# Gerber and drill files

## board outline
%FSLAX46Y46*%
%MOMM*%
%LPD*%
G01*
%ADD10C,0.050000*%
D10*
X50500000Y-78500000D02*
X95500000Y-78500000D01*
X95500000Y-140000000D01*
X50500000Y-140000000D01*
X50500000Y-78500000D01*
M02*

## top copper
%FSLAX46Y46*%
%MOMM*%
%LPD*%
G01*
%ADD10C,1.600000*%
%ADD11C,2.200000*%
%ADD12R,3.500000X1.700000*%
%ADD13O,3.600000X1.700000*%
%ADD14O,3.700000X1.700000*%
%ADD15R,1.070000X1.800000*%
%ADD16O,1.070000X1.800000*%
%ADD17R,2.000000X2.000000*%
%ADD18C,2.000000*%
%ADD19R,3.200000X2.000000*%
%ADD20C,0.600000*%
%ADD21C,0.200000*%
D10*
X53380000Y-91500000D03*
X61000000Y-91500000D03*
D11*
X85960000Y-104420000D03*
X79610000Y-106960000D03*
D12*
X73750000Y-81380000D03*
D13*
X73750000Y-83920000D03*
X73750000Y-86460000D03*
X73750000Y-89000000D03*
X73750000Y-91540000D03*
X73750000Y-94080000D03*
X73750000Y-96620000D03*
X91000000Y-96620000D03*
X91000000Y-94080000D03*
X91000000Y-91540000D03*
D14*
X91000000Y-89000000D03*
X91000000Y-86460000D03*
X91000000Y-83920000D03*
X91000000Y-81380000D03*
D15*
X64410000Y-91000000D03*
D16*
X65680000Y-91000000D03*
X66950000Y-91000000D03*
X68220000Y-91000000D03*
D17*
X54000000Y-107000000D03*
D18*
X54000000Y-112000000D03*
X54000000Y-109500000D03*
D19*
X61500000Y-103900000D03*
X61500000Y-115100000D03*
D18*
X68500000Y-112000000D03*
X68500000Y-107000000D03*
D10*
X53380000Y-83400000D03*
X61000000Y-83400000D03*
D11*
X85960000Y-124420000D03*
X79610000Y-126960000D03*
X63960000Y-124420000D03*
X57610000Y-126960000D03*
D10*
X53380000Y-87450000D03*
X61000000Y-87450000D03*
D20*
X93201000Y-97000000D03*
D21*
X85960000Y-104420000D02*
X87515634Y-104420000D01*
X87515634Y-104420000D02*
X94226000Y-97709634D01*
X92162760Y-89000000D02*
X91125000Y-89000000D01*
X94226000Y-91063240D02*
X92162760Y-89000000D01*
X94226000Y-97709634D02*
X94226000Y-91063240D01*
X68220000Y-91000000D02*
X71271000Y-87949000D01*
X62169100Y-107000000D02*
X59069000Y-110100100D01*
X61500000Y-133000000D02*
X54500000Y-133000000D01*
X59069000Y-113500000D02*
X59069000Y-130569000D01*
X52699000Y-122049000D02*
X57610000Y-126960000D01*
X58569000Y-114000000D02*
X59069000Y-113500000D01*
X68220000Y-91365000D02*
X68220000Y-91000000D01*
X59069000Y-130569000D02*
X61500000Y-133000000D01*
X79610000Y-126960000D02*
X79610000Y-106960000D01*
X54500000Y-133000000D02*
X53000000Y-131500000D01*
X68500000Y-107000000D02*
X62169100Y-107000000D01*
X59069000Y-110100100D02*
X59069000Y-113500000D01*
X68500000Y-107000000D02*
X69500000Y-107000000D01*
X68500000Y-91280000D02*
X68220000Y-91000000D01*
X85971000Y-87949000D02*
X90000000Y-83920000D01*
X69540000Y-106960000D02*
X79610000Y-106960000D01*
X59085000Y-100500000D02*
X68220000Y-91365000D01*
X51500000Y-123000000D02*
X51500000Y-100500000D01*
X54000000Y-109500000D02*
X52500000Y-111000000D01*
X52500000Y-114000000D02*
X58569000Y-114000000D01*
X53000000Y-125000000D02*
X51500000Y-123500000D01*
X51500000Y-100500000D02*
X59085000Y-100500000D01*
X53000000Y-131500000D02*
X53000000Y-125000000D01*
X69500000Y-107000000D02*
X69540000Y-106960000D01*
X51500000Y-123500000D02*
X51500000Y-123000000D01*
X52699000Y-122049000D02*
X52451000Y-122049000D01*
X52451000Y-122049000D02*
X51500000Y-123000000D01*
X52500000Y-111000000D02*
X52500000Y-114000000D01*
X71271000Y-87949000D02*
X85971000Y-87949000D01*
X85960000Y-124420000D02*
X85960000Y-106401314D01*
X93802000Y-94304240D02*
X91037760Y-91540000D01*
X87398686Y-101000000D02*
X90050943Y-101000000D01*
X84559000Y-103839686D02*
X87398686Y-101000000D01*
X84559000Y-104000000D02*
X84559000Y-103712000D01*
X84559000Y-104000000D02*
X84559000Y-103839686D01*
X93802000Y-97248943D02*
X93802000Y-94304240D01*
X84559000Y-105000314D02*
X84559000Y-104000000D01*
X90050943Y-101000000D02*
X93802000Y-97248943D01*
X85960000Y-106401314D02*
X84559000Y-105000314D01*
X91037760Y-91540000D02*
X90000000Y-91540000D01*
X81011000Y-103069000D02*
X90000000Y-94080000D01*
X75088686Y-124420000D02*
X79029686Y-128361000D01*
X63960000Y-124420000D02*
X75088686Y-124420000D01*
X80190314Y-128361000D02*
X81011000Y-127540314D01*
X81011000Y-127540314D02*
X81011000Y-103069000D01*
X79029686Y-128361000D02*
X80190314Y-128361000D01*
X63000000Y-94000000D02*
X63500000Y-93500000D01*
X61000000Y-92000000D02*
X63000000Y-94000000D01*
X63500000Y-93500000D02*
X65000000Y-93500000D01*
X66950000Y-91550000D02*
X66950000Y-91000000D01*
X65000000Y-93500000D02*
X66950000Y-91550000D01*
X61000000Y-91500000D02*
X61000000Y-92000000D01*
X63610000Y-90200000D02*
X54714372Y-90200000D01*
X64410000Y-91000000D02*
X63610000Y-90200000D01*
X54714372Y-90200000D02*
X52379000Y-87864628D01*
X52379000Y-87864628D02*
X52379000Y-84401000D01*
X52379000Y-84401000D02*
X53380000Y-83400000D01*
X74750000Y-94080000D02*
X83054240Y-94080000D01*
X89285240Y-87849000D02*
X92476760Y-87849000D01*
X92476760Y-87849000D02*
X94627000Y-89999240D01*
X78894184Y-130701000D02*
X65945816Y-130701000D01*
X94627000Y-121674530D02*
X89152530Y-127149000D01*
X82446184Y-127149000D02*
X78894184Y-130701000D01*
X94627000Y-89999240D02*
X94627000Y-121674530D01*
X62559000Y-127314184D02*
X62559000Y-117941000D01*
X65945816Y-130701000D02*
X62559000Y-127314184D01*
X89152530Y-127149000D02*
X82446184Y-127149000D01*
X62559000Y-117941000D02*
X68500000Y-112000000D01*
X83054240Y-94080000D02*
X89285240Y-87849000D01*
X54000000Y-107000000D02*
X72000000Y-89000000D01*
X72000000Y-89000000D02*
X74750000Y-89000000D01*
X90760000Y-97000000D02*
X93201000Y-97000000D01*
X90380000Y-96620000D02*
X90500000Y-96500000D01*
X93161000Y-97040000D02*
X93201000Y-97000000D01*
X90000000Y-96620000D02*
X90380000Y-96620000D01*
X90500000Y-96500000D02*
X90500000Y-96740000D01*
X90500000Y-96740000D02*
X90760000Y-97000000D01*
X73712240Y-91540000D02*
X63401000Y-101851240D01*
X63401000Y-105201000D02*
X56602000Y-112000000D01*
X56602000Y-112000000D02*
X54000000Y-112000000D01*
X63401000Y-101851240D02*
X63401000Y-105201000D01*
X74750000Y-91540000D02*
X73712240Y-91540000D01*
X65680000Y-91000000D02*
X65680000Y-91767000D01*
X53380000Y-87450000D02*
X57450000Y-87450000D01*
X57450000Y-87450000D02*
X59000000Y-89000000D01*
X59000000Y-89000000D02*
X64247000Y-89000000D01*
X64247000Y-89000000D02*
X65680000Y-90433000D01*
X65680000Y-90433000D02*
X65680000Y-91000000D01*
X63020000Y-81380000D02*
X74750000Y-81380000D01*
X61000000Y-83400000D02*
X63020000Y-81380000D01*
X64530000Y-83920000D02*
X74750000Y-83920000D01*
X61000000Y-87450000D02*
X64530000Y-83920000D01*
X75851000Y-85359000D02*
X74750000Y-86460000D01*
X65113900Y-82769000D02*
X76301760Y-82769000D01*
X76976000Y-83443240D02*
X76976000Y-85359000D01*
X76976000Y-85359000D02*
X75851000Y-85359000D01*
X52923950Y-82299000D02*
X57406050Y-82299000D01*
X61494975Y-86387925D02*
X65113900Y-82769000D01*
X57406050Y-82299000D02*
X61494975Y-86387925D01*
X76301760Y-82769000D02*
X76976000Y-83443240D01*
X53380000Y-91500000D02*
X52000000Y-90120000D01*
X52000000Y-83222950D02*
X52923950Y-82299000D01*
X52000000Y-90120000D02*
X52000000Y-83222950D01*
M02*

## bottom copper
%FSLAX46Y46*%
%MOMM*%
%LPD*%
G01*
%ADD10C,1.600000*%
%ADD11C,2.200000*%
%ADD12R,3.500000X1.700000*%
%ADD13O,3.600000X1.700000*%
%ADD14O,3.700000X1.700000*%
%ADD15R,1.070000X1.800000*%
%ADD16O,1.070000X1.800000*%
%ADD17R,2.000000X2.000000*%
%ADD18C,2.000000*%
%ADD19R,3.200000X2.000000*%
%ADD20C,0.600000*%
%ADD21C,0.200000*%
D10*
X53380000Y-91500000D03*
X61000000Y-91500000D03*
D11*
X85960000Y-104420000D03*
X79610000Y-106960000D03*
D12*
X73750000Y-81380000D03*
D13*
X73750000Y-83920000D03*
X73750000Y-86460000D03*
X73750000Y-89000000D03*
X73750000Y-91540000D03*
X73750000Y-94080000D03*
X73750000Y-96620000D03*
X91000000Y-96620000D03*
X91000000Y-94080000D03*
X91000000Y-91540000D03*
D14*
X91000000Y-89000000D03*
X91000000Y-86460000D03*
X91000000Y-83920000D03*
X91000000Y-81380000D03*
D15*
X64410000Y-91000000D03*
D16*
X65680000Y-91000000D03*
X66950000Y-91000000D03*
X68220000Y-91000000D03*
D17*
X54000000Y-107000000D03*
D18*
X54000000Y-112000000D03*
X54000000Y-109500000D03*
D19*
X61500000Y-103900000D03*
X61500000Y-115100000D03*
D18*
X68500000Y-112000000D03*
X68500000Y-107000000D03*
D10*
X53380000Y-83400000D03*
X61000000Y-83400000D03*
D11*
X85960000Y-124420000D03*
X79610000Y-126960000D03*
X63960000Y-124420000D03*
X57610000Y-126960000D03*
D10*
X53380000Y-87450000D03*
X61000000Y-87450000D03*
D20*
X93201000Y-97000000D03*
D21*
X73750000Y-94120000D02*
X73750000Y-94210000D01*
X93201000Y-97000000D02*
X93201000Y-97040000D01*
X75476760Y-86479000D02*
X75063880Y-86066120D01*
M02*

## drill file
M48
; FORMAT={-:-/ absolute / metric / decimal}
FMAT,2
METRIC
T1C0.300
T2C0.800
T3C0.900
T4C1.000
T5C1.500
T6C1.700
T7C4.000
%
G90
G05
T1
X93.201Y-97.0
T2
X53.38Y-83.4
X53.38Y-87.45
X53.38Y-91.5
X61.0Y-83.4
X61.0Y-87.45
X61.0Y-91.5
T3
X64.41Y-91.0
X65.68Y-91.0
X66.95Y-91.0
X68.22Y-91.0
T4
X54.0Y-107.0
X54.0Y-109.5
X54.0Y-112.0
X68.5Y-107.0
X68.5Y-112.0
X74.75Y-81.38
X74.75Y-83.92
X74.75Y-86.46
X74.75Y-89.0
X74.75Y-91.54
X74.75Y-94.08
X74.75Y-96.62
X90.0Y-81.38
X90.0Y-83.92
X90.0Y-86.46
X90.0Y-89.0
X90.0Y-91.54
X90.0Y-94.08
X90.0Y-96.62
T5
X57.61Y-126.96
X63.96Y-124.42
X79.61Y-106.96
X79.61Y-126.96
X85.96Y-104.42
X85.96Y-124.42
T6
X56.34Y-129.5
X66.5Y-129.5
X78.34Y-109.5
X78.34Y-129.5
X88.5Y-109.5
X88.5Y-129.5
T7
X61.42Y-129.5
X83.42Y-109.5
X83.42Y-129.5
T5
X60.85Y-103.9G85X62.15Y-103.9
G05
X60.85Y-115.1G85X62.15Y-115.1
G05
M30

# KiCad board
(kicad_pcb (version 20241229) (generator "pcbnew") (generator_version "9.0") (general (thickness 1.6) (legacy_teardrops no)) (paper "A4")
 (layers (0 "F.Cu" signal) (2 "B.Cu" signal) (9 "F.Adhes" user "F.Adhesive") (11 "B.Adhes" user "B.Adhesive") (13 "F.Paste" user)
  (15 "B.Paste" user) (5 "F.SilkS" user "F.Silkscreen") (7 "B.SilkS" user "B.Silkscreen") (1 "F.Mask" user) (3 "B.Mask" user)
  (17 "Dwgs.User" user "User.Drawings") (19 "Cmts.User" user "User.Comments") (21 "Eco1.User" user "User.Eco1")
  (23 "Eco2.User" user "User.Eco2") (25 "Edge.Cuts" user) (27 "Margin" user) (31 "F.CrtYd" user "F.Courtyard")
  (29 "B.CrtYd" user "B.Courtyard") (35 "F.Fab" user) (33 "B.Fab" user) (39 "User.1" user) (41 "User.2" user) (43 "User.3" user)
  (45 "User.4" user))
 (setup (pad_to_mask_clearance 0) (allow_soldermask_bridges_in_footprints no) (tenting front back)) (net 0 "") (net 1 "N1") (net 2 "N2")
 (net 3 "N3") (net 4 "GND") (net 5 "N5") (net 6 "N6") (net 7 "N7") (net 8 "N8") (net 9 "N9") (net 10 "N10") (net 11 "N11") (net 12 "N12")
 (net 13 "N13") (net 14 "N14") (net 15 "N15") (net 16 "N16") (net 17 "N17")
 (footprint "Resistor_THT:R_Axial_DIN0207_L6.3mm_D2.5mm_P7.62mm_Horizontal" (layer "F.Cu") (at 53.38 91.5)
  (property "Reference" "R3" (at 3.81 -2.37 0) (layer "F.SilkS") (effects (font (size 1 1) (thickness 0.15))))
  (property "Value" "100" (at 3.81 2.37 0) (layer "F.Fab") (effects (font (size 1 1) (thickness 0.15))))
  (pad "1" thru_hole circle (at 0 0) (size 1.6 1.6) (drill 0.8) (layers "*.Cu" "*.Mask") (remove_unused_layers no) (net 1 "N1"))
  (pad "2" thru_hole circle (at 7.62 0) (size 1.6 1.6) (drill 0.8) (layers "*.Cu" "*.Mask") (remove_unused_layers no) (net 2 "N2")))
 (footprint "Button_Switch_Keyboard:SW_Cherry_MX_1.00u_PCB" (layer "F.Cu") (at 85.96 104.42)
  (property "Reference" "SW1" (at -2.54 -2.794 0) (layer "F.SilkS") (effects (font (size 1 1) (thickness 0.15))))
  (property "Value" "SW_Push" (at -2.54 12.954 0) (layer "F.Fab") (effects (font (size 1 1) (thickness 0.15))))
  (pad "" np_thru_hole circle (at -7.62 5.08) (size 1.7 1.7) (drill 1.7) (layers "*.Cu" "*.Mask"))
  (pad "" np_thru_hole circle (at -2.54 5.08) (size 4 4) (drill 4) (layers "*.Cu" "*.Mask"))
  (pad "" np_thru_hole circle (at 2.54 5.08) (size 1.7 1.7) (drill 1.7) (layers "*.Cu" "*.Mask"))
  (pad "1" thru_hole circle (at 0 0) (size 2.2 2.2) (drill 1.5) (layers "*.Cu" "*.Mask") (remove_unused_layers no) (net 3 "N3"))
  (pad "2" thru_hole circle (at -6.35 2.54) (size 2.2 2.2) (drill 1.5) (layers "*.Cu" "*.Mask") (remove_unused_layers no) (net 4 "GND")))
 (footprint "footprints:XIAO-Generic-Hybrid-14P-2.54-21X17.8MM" (layer "F.Cu") (at 82.375 89)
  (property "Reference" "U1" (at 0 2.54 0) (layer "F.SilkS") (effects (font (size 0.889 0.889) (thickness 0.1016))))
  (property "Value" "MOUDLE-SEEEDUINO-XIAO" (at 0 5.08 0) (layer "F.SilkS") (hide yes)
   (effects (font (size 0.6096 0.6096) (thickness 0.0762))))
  (pad "1" thru_hole rect (at -7.625 -7.62) (size 3.5 1.7) (drill 1 (offset -1 0)) (layers "*.Cu" "*.Mask") (remove_unused_layers no)
   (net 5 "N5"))
  (pad "2" thru_hole oval (at -7.625 -5.08) (size 3.6 1.7) (drill 1 (offset -1 0)) (layers "*.Cu" "*.Mask") (remove_unused_layers no)
   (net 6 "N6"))
  (pad "3" thru_hole oval (at -7.625 -2.54) (size 3.6 1.7) (drill 1 (offset -1 0)) (layers "*.Cu" "*.Mask") (remove_unused_layers no)
   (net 1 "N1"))
  (pad "4" thru_hole oval (at -7.625 0) (size 3.6 1.7) (drill 1 (offset -1 0)) (layers "*.Cu" "*.Mask") (remove_unused_layers no)
   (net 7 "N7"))
  (pad "5" thru_hole oval (at -7.625 2.54) (size 3.6 1.7) (drill 1 (offset -1 0)) (layers "*.Cu" "*.Mask") (remove_unused_layers no)
   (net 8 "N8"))
  (pad "6" thru_hole oval (at -7.625 5.08 180) (size 3.6 1.7) (drill 1 (offset 1 0)) (layers "*.Cu" "*.Mask") (remove_unused_layers no)
   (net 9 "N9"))
  (pad "7" thru_hole oval (at -7.625 7.62) (size 3.6 1.7) (drill 1 (offset -1 0)) (layers "*.Cu" "*.Mask") (remove_unused_layers no)
   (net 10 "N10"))
  (pad "8" thru_hole oval (at 7.625 7.62) (size 3.6 1.7) (drill 1 (offset 1 0)) (layers "*.Cu" "*.Mask") (remove_unused_layers no)
   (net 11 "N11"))
  (pad "9" thru_hole oval (at 7.625 5.08) (size 3.6 1.7) (drill 1 (offset 1 0)) (layers "*.Cu" "*.Mask") (remove_unused_layers no)
   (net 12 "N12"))
  (pad "10" thru_hole oval (at 7.625 2.54) (size 3.6 1.7) (drill 1 (offset 1 0)) (layers "*.Cu" "*.Mask") (remove_unused_layers no)
   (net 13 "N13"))
  (pad "11" thru_hole oval (at 7.625 0) (size 3.7 1.7) (drill 1 (offset 1 0)) (layers "*.Cu" "*.Mask") (remove_unused_layers no)
   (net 3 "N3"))
  (pad "12" thru_hole oval (at 7.625 -2.54) (size 3.7 1.7) (drill 1 (offset 1 0)) (layers "*.Cu" "*.Mask") (remove_unused_layers no)
   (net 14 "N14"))
  (pad "13" thru_hole oval (at 7.625 -5.08) (size 3.7 1.7) (drill 1 (offset 1 0)) (layers "*.Cu" "*.Mask") (remove_unused_layers no)
   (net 4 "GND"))
  (pad "14" thru_hole oval (at 7.625 -7.62) (size 3.7 1.7) (drill 1 (offset 1 0)) (layers "*.Cu" "*.Mask") (remove_unused_layers no)
   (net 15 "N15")))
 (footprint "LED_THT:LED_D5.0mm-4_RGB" (layer "F.Cu") (at 64.41 91)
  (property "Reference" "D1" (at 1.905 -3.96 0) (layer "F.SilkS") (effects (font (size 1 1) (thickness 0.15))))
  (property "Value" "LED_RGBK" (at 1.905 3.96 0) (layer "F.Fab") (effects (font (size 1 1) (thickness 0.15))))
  (pad "1" thru_hole rect (at 0 0) (size 1.07 1.8) (drill 0.9) (layers "*.Cu" "*.Mask") (remove_unused_layers no) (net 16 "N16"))
  (pad "2" thru_hole oval (at 1.27 0) (size 1.07 1.8) (drill 0.9) (layers "*.Cu" "*.Mask") (remove_unused_layers no) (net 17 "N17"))
  (pad "3" thru_hole oval (at 2.54 0) (size 1.07 1.8) (drill 0.9) (layers "*.Cu" "*.Mask") (remove_unused_layers no) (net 2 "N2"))
  (pad "4" thru_hole oval (at 3.81 0) (size 1.07 1.8) (drill 0.9) (layers "*.Cu" "*.Mask") (remove_unused_layers no) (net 4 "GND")))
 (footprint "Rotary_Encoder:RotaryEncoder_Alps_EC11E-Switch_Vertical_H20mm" (layer "F.Cu") (at 54 107)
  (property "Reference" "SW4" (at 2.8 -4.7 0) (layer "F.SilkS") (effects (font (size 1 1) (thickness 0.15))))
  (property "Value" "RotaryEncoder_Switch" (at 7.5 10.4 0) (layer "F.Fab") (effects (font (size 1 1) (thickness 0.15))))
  (pad "A" thru_hole rect (at 0 0) (size 2 2) (drill 1) (layers "*.Cu" "*.Mask") (remove_unused_layers no) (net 7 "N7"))
  (pad "B" thru_hole circle (at 0 5) (size 2 2) (drill 1) (layers "*.Cu" "*.Mask") (remove_unused_layers no) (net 8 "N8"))
  (pad "C" thru_hole circle (at 0 2.5) (size 2 2) (drill 1) (layers "*.Cu" "*.Mask") (remove_unused_layers no) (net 4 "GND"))
  (pad "MP" thru_hole rect (at 7.5 -3.1) (size 3.2 2) (drill oval 2.8 1.5) (layers "*.Cu" "*.Mask") (remove_unused_layers no))
  (pad "MP" thru_hole rect (at 7.5 8.1) (size 3.2 2) (drill oval 2.8 1.5) (layers "*.Cu" "*.Mask") (remove_unused_layers no))
  (pad "S1" thru_hole circle (at 14.5 5) (size 2 2) (drill 1) (layers "*.Cu" "*.Mask") (remove_unused_layers no) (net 9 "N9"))
  (pad "S2" thru_hole circle (at 14.5 0) (size 2 2) (drill 1) (layers "*.Cu" "*.Mask") (remove_unused_layers no) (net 4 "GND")))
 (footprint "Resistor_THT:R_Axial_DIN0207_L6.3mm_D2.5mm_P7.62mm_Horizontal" (layer "F.Cu") (at 53.38 83.4)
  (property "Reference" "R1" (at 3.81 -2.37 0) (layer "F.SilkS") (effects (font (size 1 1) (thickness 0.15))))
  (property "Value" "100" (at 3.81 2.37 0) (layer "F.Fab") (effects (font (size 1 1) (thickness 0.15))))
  (pad "1" thru_hole circle (at 0 0) (size 1.6 1.6) (drill 0.8) (layers "*.Cu" "*.Mask") (remove_unused_layers no) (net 16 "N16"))
  (pad "2" thru_hole circle (at 7.62 0) (size 1.6 1.6) (drill 0.8) (layers "*.Cu" "*.Mask") (remove_unused_layers no) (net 5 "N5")))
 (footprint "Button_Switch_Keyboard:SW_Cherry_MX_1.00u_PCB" (layer "F.Cu") (at 85.96 124.42)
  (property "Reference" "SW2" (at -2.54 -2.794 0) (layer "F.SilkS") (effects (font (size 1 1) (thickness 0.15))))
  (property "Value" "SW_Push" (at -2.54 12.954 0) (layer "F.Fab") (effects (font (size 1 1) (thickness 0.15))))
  (pad "" np_thru_hole circle (at -7.62 5.08) (size 1.7 1.7) (drill 1.7) (layers "*.Cu" "*.Mask"))
  (pad "" np_thru_hole circle (at -2.54 5.08) (size 4 4) (drill 4) (layers "*.Cu" "*.Mask"))
  (pad "" np_thru_hole circle (at 2.54 5.08) (size 1.7 1.7) (drill 1.7) (layers "*.Cu" "*.Mask"))
  (pad "1" thru_hole circle (at 0 0) (size 2.2 2.2) (drill 1.5) (layers "*.Cu" "*.Mask") (remove_unused_layers no) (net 13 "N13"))
  (pad "2" thru_hole circle (at -6.35 2.54) (size 2.2 2.2) (drill 1.5) (layers "*.Cu" "*.Mask") (remove_unused_layers no) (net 4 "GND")))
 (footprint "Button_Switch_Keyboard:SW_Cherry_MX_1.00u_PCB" (layer "F.Cu") (at 63.96 124.42)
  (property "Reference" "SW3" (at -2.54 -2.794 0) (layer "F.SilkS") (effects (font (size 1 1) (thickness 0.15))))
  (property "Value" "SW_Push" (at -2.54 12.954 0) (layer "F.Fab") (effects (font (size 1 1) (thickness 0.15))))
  (pad "" np_thru_hole circle (at -7.62 5.08) (size 1.7 1.7) (drill 1.7) (layers "*.Cu" "*.Mask"))
  (pad "" np_thru_hole circle (at -2.54 5.08) (size 4 4) (drill 4) (layers "*.Cu" "*.Mask"))
  (pad "" np_thru_hole circle (at 2.54 5.08) (size 1.7 1.7) (drill 1.7) (layers "*.Cu" "*.Mask"))
  (pad "1" thru_hole circle (at 0 0) (size 2.2 2.2) (drill 1.5) (layers "*.Cu" "*.Mask") (remove_unused_layers no) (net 12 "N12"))
  (pad "2" thru_hole circle (at -6.35 2.54) (size 2.2 2.2) (drill 1.5) (layers "*.Cu" "*.Mask") (remove_unused_layers no) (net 4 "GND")))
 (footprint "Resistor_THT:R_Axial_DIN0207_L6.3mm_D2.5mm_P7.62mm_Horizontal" (layer "F.Cu") (at 53.38 87.45)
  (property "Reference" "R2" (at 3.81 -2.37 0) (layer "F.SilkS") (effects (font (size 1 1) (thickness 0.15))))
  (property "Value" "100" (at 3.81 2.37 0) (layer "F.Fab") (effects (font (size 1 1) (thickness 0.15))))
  (pad "1" thru_hole circle (at 0 0) (size 1.6 1.6) (drill 0.8) (layers "*.Cu" "*.Mask") (remove_unused_layers no) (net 17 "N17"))
  (pad "2" thru_hole circle (at 7.62 0) (size 1.6 1.6) (drill 0.8) (layers "*.Cu" "*.Mask") (remove_unused_layers no) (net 6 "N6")))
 (gr_rect (start 50.5 78.5) (end 95.5 140) (stroke (width 0.05) (type default)) (fill no) (layer "Edge.Cuts"))
 (segment (start 85.96 104.42) (end 87.515634 104.42) (width 0.2) (layer "F.Cu") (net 3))
 (segment (start 87.515634 104.42) (end 94.226 97.709634) (width 0.2) (layer "F.Cu") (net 3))
 (segment (start 92.16276 89) (end 91.125 89) (width 0.2) (layer "F.Cu") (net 3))
 (segment (start 94.226 91.06324) (end 92.16276 89) (width 0.2) (layer "F.Cu") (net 3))
 (segment (start 94.226 97.709634) (end 94.226 91.06324) (width 0.2) (layer "F.Cu") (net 3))
 (segment (start 68.22 91) (end 71.271 87.949) (width 0.2) (layer "F.Cu") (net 4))
 (segment (start 62.1691 107) (end 59.069 110.1001) (width 0.2) (layer "F.Cu") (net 4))
 (segment (start 61.5 133) (end 54.5 133) (width 0.2) (layer "F.Cu") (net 4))
 (segment (start 59.069 113.5) (end 59.069 130.569) (width 0.2) (layer "F.Cu") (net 4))
 (segment (start 52.699 122.049) (end 57.61 126.96) (width 0.2) (layer "F.Cu") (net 4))
 (segment (start 58.569 114) (end 59.069 113.5) (width 0.2) (layer "F.Cu") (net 4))
 (segment (start 68.22 91.365) (end 68.22 91) (width 0.2) (layer "F.Cu") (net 4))
 (segment (start 59.069 130.569) (end 61.5 133) (width 0.2) (layer "F.Cu") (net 4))
 (segment (start 79.61 126.96) (end 79.61 106.96) (width 0.2) (layer "F.Cu") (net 4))
 (segment (start 54.5 133) (end 53 131.5) (width 0.2) (layer "F.Cu") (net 4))
 (segment (start 68.5 107) (end 62.1691 107) (width 0.2) (layer "F.Cu") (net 4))
 (segment (start 59.069 110.1001) (end 59.069 113.5) (width 0.2) (layer "F.Cu") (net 4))
 (segment (start 68.5 107) (end 69.5 107) (width 0.2) (layer "F.Cu") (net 4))
 (segment (start 68.5 91.28) (end 68.22 91) (width 0.2) (layer "F.Cu") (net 4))
 (segment (start 85.971 87.949) (end 90 83.92) (width 0.2) (layer "F.Cu") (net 4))
 (segment (start 69.54 106.96) (end 79.61 106.96) (width 0.2) (layer "F.Cu") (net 4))
 (segment (start 59.085 100.5) (end 68.22 91.365) (width 0.2) (layer "F.Cu") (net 4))
 (segment (start 51.5 123) (end 51.5 100.5) (width 0.2) (layer "F.Cu") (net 4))
 (segment (start 54 109.5) (end 52.5 111) (width 0.2) (layer "F.Cu") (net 4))
 (segment (start 52.5 114) (end 58.569 114) (width 0.2) (layer "F.Cu") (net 4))
 (segment (start 53 125) (end 51.5 123.5) (width 0.2) (layer "F.Cu") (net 4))
 (segment (start 51.5 100.5) (end 59.085 100.5) (width 0.2) (layer "F.Cu") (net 4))
 (segment (start 53 131.5) (end 53 125) (width 0.2) (layer "F.Cu") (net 4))
 (segment (start 69.5 107) (end 69.54 106.96) (width 0.2) (layer "F.Cu") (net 4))
 (segment (start 51.5 123.5) (end 51.5 123) (width 0.2) (layer "F.Cu") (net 4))
 (segment (start 52.699 122.049) (end 52.451 122.049) (width 0.2) (layer "F.Cu") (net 4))
 (segment (start 52.451 122.049) (end 51.5 123) (width 0.2) (layer "F.Cu") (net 4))
 (segment (start 52.5 111) (end 52.5 114) (width 0.2) (layer "F.Cu") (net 4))
 (segment (start 71.271 87.949) (end 85.971 87.949) (width 0.2) (layer "F.Cu") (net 4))
 (segment (start 85.96 124.42) (end 85.96 106.401314) (width 0.2) (layer "F.Cu") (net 13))
 (segment (start 93.802 94.30424) (end 91.03776 91.54) (width 0.2) (layer "F.Cu") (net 13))
 (segment (start 87.398686 101) (end 90.050943 101) (width 0.2) (layer "F.Cu") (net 13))
 (segment (start 84.559 103.839686) (end 87.398686 101) (width 0.2) (layer "F.Cu") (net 13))
 (segment (start 84.559 104) (end 84.559 103.712) (width 0.2) (layer "F.Cu") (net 13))
 (segment (start 84.559 104) (end 84.559 103.839686) (width 0.2) (layer "F.Cu") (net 13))
 (segment (start 93.802 97.248943) (end 93.802 94.30424) (width 0.2) (layer "F.Cu") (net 13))
 (segment (start 84.559 105.000314) (end 84.559 104) (width 0.2) (layer "F.Cu") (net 13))
 (segment (start 90.050943 101) (end 93.802 97.248943) (width 0.2) (layer "F.Cu") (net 13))
 (segment (start 85.96 106.401314) (end 84.559 105.000314) (width 0.2) (layer "F.Cu") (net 13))
 (segment (start 91.03776 91.54) (end 90 91.54) (width 0.2) (layer "F.Cu") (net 13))
 (segment (start 81.011 103.069) (end 90 94.08) (width 0.2) (layer "F.Cu") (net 12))
 (segment (start 75.088686 124.42) (end 79.029686 128.361) (width 0.2) (layer "F.Cu") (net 12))
 (segment (start 63.96 124.42) (end 75.088686 124.42) (width 0.2) (layer "F.Cu") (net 12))
 (segment (start 80.190314 128.361) (end 81.011 127.540314) (width 0.2) (layer "F.Cu") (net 12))
 (segment (start 81.011 127.540314) (end 81.011 103.069) (width 0.2) (layer "F.Cu") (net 12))
 (segment (start 79.029686 128.361) (end 80.190314 128.361) (width 0.2) (layer "F.Cu") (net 12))
 (segment (start 63 94) (end 63.5 93.5) (width 0.2) (layer "F.Cu") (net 2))
 (segment (start 61 92) (end 63 94) (width 0.2) (layer "F.Cu") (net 2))
 (segment (start 63.5 93.5) (end 65 93.5) (width 0.2) (layer "F.Cu") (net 2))
 (segment (start 66.95 91.55) (end 66.95 91) (width 0.2) (layer "F.Cu") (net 2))
 (segment (start 65 93.5) (end 66.95 91.55) (width 0.2) (layer "F.Cu") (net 2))
 (segment (start 61 91.5) (end 61 92) (width 0.2) (layer "F.Cu") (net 2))
 (segment (start 63.61 90.2) (end 54.714372 90.2) (width 0.2) (layer "F.Cu") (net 16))
 (segment (start 64.41 91) (end 63.61 90.2) (width 0.2) (layer "F.Cu") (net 16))
 (segment (start 54.714372 90.2) (end 52.379 87.864628) (width 0.2) (layer "F.Cu") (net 16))
 (segment (start 52.379 87.864628) (end 52.379 84.401) (width 0.2) (layer "F.Cu") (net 16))
 (segment (start 52.379 84.401) (end 53.38 83.4) (width 0.2) (layer "F.Cu") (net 16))
 (segment (start 74.75 94.08) (end 83.05424 94.08) (width 0.2) (layer "F.Cu") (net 9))
 (segment (start 89.28524 87.849) (end 92.47676 87.849) (width 0.2) (layer "F.Cu") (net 9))
 (segment (start 92.47676 87.849) (end 94.627 89.99924) (width 0.2) (layer "F.Cu") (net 9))
 (segment (start 78.894184 130.701) (end 65.945816 130.701) (width 0.2) (layer "F.Cu") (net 9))
 (segment (start 94.627 121.67453) (end 89.15253 127.149) (width 0.2) (layer "F.Cu") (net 9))
 (segment (start 82.446184 127.149) (end 78.894184 130.701) (width 0.2) (layer "F.Cu") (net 9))
 (segment (start 94.627 89.99924) (end 94.627 121.67453) (width 0.2) (layer "F.Cu") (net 9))
 (segment (start 62.559 127.314184) (end 62.559 117.941) (width 0.2) (layer "F.Cu") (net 9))
 (segment (start 65.945816 130.701) (end 62.559 127.314184) (width 0.2) (layer "F.Cu") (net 9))
 (segment (start 89.15253 127.149) (end 82.446184 127.149) (width 0.2) (layer "F.Cu") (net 9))
 (segment (start 62.559 117.941) (end 68.5 112) (width 0.2) (layer "F.Cu") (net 9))
 (segment (start 83.05424 94.08) (end 89.28524 87.849) (width 0.2) (layer "F.Cu") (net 9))
 (segment (start 73.75 94.12) (end 73.75 94.21) (width 0.2) (layer "B.Cu") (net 9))
 (segment (start 54 107) (end 72 89) (width 0.2) (layer "F.Cu") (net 7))
 (segment (start 72 89) (end 74.75 89) (width 0.2) (layer "F.Cu") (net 7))
 (segment (start 90.76 97) (end 93.201 97) (width 0.2) (layer "F.Cu") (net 11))
 (segment (start 90.38 96.62) (end 90.5 96.5) (width 0.2) (layer "F.Cu") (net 11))
 (segment (start 93.161 97.04) (end 93.201 97) (width 0.2) (layer "F.Cu") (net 11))
 (segment (start 90 96.62) (end 90.38 96.62) (width 0.2) (layer "F.Cu") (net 11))
 (segment (start 90.5 96.5) (end 90.5 96.74) (width 0.2) (layer "F.Cu") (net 11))
 (segment (start 90.5 96.74) (end 90.76 97) (width 0.2) (layer "F.Cu") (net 11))
 (via (at 93.201 97) (size 0.6) (drill 0.3) (layers "F.Cu" "B.Cu") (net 11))
 (segment (start 93.201 97) (end 93.201 97.04) (width 0.2) (layer "B.Cu") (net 11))
 (segment (start 73.71224 91.54) (end 63.401 101.85124) (width 0.2) (layer "F.Cu") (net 8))
 (segment (start 63.401 105.201) (end 56.602 112) (width 0.2) (layer "F.Cu") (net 8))
 (segment (start 56.602 112) (end 54 112) (width 0.2) (layer "F.Cu") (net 8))
 (segment (start 63.401 101.85124) (end 63.401 105.201) (width 0.2) (layer "F.Cu") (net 8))
 (segment (start 74.75 91.54) (end 73.71224 91.54) (width 0.2) (layer "F.Cu") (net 8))
 (segment (start 65.68 91) (end 65.68 91.767) (width 0.2) (layer "F.Cu") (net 17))
 (segment (start 53.38 87.45) (end 57.45 87.45) (width 0.2) (layer "F.Cu") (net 17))
 (segment (start 57.45 87.45) (end 59 89) (width 0.2) (layer "F.Cu") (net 17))
 (segment (start 59 89) (end 64.247 89) (width 0.2) (layer "F.Cu") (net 17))
 (segment (start 64.247 89) (end 65.68 90.433) (width 0.2) (layer "F.Cu") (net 17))
 (segment (start 65.68 90.433) (end 65.68 91) (width 0.2) (layer "F.Cu") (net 17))
 (segment (start 63.02 81.38) (end 74.75 81.38) (width 0.2) (layer "F.Cu") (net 5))
 (segment (start 61 83.4) (end 63.02 81.38) (width 0.2) (layer "F.Cu") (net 5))
 (segment (start 64.53 83.92) (end 74.75 83.92) (width 0.2) (layer "F.Cu") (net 6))
 (segment (start 61 87.45) (end 64.53 83.92) (width 0.2) (layer "F.Cu") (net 6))
 (segment (start 75.851 85.359) (end 74.75 86.46) (width 0.2) (layer "F.Cu") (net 1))
 (segment (start 65.1139 82.769) (end 76.30176 82.769) (width 0.2) (layer "F.Cu") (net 1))
 (segment (start 76.976 83.44324) (end 76.976 85.359) (width 0.2) (layer "F.Cu") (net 1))
 (segment (start 76.976 85.359) (end 75.851 85.359) (width 0.2) (layer "F.Cu") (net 1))
 (segment (start 52.92395 82.299) (end 57.40605 82.299) (width 0.2) (layer "F.Cu") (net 1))
 (segment (start 61.494975 86.387925) (end 65.1139 82.769) (width 0.2) (layer "F.Cu") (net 1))
 (segment (start 57.40605 82.299) (end 61.494975 86.387925) (width 0.2) (layer "F.Cu") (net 1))
 (segment (start 76.30176 82.769) (end 76.976 83.44324) (width 0.2) (layer "F.Cu") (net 1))
 (segment (start 53.38 91.5) (end 52 90.12) (width 0.2) (layer "F.Cu") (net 1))
 (segment (start 52 83.22295) (end 52.92395 82.299) (width 0.2) (layer "F.Cu") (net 1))
 (segment (start 52 90.12) (end 52 83.22295) (width 0.2) (layer "F.Cu") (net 1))
 (segment (start 75.47676 86.479) (end 75.06388 86.06612) (width 0.2) (layer "B.Cu") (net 1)))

